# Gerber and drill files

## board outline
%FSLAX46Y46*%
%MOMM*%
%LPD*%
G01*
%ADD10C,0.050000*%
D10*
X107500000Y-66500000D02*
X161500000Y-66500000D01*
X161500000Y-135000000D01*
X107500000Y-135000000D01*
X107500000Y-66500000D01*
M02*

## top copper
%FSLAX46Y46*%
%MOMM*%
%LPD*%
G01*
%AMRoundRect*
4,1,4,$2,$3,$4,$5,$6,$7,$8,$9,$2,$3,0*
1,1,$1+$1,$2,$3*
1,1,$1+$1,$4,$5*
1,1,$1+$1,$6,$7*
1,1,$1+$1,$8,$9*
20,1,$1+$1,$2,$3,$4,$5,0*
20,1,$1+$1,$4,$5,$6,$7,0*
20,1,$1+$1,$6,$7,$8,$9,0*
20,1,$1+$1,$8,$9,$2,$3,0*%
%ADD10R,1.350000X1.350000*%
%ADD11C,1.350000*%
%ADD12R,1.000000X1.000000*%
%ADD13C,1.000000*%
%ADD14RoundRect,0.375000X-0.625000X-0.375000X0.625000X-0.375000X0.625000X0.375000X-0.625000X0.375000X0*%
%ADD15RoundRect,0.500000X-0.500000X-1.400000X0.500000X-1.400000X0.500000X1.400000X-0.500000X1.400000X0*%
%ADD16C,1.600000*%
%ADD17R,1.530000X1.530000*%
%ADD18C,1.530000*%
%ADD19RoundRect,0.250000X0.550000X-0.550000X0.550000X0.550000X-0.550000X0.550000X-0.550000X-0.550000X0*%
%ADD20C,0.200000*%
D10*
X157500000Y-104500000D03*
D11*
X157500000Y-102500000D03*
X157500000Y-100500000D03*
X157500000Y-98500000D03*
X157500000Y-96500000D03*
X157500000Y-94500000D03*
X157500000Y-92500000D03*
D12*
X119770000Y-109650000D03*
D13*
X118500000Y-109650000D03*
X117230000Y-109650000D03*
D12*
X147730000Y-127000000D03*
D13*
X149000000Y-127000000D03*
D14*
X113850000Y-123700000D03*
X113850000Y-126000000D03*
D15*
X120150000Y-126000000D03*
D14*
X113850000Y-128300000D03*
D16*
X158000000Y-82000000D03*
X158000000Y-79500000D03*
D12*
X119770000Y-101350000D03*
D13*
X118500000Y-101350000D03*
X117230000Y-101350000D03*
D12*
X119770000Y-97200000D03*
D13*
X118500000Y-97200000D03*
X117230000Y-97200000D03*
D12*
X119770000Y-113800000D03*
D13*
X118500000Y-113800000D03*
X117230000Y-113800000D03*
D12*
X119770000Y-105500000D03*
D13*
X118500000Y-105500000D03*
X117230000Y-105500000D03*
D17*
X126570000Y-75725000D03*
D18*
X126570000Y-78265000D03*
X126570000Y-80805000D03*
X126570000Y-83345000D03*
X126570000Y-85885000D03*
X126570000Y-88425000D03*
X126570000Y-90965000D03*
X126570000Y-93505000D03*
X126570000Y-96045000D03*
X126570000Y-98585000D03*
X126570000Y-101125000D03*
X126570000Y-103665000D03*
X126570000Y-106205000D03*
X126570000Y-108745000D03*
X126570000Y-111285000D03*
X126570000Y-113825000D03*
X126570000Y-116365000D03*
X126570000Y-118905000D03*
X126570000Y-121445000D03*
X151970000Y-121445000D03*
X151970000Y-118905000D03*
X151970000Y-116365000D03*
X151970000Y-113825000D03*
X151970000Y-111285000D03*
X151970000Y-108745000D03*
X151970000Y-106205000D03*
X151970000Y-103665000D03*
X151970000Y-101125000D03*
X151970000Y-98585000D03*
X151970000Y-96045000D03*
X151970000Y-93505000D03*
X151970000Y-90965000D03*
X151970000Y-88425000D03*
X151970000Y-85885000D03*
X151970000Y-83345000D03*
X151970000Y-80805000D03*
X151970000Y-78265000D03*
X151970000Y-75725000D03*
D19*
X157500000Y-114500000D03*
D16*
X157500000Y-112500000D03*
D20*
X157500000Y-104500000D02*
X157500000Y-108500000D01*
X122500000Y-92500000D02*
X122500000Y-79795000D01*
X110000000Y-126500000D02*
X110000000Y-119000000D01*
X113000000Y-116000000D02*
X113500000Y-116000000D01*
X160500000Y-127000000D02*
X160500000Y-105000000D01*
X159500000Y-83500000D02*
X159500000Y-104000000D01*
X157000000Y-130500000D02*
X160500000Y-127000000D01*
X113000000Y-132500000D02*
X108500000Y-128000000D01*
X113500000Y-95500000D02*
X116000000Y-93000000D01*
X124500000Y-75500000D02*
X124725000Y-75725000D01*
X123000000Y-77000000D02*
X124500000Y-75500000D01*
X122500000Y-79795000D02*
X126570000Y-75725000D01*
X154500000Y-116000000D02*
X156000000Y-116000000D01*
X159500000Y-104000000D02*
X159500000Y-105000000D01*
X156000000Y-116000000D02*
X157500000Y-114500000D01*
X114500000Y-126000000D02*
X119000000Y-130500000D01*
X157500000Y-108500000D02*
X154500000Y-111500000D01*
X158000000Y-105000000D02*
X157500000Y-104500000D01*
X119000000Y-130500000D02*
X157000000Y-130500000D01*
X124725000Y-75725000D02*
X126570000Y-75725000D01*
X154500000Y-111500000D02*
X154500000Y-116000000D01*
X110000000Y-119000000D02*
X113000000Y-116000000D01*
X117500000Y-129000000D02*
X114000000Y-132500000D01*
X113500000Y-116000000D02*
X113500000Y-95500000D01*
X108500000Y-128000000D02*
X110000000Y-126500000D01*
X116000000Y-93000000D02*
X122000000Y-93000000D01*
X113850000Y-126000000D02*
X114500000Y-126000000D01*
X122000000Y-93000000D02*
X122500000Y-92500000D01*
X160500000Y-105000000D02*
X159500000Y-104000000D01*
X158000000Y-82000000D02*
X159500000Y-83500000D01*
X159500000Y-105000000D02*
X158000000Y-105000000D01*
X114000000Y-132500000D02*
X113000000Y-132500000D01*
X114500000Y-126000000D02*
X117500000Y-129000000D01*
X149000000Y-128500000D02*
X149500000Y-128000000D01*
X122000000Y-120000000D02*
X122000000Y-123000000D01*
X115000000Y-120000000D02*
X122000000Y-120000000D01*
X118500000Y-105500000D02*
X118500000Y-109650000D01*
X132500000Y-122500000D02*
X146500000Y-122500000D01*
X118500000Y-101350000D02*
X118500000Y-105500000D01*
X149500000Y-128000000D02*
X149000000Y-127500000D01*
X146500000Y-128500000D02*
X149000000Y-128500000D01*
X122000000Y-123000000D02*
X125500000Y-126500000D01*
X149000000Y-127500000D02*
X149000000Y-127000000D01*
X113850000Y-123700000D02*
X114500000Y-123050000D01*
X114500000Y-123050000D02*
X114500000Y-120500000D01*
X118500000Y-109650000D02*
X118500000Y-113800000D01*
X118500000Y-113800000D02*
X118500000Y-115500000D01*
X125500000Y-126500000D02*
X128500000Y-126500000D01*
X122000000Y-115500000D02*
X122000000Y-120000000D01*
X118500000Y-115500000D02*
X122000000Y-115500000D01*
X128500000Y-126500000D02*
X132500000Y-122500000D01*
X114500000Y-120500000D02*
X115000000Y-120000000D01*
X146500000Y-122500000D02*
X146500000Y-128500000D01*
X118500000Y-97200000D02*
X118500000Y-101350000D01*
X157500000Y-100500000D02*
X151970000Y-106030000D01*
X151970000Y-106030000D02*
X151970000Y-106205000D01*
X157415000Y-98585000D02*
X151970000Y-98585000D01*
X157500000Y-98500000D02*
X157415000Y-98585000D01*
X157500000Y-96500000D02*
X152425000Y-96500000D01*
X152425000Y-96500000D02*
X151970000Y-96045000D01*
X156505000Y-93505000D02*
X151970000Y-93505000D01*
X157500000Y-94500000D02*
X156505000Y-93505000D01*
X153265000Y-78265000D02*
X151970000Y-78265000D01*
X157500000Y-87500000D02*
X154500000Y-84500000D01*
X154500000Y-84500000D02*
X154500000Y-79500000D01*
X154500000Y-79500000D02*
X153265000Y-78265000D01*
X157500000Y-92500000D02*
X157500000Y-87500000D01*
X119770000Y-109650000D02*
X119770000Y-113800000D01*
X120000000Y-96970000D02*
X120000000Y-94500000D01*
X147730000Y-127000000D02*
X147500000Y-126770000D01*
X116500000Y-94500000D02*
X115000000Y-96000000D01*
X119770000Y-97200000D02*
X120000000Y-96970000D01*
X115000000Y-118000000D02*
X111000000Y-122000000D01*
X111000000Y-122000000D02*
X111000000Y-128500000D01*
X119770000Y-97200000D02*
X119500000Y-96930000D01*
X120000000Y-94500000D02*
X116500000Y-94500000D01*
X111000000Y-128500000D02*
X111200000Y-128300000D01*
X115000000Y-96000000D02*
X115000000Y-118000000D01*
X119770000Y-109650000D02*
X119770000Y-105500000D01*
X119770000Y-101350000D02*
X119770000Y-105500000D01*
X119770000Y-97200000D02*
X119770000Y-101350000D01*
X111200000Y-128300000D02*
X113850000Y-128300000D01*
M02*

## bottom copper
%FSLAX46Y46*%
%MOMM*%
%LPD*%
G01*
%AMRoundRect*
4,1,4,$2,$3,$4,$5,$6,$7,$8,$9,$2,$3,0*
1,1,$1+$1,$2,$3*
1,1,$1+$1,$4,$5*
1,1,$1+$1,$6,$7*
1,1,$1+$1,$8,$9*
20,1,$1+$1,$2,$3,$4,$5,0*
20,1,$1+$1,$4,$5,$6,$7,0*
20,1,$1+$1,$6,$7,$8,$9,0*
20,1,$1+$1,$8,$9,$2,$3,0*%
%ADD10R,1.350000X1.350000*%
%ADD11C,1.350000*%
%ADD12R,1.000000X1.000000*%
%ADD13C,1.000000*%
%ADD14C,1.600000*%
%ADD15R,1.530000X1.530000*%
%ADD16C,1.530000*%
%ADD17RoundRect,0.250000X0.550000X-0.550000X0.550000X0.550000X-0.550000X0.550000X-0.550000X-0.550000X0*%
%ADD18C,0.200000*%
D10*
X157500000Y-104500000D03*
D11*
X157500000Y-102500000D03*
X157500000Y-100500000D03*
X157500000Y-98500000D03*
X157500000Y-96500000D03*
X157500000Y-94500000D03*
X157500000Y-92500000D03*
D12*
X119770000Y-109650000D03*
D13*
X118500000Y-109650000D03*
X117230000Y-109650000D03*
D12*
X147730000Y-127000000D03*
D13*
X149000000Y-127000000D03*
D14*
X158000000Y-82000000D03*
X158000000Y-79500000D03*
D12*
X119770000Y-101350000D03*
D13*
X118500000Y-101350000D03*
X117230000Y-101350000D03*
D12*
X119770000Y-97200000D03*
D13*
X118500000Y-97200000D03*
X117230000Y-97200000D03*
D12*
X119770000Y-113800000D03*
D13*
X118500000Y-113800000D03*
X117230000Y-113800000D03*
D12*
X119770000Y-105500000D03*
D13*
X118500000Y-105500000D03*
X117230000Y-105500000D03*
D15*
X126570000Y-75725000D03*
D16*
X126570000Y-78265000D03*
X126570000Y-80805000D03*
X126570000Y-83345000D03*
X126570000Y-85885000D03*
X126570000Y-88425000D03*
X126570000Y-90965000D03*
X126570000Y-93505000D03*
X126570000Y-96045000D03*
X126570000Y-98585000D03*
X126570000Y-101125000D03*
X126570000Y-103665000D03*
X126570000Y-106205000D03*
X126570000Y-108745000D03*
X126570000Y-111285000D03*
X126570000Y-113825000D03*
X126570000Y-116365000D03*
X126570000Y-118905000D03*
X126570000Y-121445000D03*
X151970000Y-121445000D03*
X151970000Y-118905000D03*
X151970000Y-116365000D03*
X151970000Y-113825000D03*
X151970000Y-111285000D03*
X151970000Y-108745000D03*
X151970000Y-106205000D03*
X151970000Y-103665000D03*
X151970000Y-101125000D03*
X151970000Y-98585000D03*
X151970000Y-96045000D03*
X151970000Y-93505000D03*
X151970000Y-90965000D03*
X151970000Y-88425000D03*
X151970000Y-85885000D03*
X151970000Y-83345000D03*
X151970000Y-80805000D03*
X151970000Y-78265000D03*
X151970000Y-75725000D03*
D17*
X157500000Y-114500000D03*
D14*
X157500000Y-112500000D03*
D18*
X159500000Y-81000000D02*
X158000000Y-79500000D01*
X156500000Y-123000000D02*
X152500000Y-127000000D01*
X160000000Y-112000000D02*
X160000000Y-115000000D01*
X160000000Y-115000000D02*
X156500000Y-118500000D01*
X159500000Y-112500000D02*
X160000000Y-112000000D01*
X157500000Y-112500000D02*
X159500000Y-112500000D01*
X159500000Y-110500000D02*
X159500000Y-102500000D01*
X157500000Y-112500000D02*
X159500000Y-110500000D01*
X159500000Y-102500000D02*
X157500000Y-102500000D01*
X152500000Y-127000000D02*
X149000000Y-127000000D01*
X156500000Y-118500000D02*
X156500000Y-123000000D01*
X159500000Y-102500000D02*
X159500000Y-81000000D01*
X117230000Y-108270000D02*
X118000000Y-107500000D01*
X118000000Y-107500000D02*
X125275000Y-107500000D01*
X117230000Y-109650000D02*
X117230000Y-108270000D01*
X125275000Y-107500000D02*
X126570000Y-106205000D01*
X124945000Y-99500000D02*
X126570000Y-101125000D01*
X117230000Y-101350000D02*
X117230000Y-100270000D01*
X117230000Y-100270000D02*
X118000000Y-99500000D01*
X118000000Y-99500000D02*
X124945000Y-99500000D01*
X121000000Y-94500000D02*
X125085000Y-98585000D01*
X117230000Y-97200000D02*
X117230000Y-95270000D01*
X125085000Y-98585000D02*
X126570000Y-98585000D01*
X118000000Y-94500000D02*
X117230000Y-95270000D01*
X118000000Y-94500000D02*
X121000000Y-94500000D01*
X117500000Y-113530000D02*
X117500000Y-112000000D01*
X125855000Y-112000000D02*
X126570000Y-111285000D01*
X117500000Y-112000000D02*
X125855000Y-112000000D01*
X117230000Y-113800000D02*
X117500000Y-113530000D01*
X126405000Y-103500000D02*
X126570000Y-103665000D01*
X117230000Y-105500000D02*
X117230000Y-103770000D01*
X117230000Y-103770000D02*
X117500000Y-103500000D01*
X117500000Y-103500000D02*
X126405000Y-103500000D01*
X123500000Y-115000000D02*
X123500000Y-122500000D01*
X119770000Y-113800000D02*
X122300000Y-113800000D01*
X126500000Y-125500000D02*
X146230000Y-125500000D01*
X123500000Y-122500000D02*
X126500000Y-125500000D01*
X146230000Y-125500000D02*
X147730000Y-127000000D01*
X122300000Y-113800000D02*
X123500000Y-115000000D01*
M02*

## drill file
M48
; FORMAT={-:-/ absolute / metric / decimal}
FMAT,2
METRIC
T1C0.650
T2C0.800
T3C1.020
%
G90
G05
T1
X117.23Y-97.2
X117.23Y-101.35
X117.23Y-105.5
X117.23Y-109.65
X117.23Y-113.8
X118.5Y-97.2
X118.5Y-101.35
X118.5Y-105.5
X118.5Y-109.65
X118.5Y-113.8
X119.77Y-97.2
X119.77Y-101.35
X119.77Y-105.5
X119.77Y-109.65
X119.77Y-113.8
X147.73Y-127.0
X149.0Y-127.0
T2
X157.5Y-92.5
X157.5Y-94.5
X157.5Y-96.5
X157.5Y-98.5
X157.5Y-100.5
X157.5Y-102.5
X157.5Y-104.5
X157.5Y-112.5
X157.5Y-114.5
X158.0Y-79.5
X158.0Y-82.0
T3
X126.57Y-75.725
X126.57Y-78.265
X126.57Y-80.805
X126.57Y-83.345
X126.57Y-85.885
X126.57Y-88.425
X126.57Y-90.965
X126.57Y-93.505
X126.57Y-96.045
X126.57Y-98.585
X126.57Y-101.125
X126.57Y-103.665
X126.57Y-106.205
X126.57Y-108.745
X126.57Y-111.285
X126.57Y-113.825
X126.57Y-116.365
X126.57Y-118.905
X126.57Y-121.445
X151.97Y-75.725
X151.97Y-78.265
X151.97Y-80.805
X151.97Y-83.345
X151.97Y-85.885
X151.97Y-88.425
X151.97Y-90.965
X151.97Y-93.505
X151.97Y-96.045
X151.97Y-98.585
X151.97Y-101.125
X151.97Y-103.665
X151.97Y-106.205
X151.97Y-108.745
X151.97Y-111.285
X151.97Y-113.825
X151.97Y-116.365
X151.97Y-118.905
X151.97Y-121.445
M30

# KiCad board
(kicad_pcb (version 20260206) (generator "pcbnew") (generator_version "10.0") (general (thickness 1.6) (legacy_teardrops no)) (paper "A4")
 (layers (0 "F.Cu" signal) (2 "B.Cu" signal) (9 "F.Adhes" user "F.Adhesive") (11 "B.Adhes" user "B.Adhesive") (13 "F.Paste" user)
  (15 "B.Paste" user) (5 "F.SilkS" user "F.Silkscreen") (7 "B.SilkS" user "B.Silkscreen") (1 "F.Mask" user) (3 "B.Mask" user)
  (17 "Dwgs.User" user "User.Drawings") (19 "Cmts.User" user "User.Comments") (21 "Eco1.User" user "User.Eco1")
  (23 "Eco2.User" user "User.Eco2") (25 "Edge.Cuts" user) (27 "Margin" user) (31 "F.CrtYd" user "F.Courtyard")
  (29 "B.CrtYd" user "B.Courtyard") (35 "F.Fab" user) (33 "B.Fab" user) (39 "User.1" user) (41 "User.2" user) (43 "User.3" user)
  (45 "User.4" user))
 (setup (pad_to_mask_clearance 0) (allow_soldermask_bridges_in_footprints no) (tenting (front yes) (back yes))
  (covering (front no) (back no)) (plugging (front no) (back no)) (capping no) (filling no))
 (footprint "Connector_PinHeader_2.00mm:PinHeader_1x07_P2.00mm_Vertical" (layer "F.Cu") (at 157.5 104.5 180)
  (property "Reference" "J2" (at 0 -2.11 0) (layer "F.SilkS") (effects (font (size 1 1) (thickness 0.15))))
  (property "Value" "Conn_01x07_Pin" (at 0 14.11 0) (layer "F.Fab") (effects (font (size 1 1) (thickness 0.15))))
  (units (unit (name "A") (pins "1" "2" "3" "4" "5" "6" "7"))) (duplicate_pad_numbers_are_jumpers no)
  (pad "1" thru_hole rect (at 0 0 180) (size 1.35 1.35) (drill 0.8) (layers "*.Cu" "*.Mask") (remove_unused_layers no) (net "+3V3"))
  (pad "2" thru_hole circle (at 0 2 180) (size 1.35 1.35) (drill 0.8) (layers "*.Cu" "*.Mask") (remove_unused_layers no) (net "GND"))
  (pad "3" thru_hole circle (at 0 4 180) (size 1.35 1.35) (drill 0.8) (layers "*.Cu" "*.Mask") (remove_unused_layers no)
   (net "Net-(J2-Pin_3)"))
  (pad "4" thru_hole circle (at 0 6 180) (size 1.35 1.35) (drill 0.8) (layers "*.Cu" "*.Mask") (remove_unused_layers no)
   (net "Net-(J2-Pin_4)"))
  (pad "5" thru_hole circle (at 0 8 180) (size 1.35 1.35) (drill 0.8) (layers "*.Cu" "*.Mask") (remove_unused_layers no)
   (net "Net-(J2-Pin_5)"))
  (pad "6" thru_hole circle (at 0 10 180) (size 1.35 1.35) (drill 0.8) (layers "*.Cu" "*.Mask") (remove_unused_layers no)
   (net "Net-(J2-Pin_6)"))
  (pad "7" thru_hole circle (at 0 12 180) (size 1.35 1.35) (drill 0.8) (layers "*.Cu" "*.Mask") (remove_unused_layers no)
   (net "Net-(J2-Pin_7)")))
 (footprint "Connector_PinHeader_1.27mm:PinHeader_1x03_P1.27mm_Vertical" (layer "F.Cu") (at 119.77 109.65 -90)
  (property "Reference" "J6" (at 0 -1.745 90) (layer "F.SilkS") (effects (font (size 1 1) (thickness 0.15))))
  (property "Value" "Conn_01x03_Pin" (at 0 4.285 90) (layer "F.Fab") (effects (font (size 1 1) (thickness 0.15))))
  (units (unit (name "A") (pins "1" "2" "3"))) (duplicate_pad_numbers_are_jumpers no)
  (pad "1" thru_hole rect (at 0 0 270) (size 1 1) (drill 0.65) (layers "*.Cu" "*.Mask") (remove_unused_layers no) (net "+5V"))
  (pad "2" thru_hole circle (at 0 1.27 270) (size 1 1) (drill 0.65) (layers "*.Cu" "*.Mask") (remove_unused_layers no) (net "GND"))
  (pad "3" thru_hole circle (at 0 2.54 270) (size 1 1) (drill 0.65) (layers "*.Cu" "*.Mask") (remove_unused_layers no)
   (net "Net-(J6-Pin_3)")))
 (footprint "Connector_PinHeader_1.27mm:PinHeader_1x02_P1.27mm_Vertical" (layer "F.Cu") (at 147.73 127 90)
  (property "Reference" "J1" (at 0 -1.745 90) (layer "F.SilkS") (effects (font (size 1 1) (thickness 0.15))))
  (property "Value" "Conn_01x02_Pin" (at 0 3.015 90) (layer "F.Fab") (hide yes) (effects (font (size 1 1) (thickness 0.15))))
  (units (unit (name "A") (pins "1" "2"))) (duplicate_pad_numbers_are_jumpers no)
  (pad "1" thru_hole rect (at 0 0 90) (size 1 1) (drill 0.65) (layers "*.Cu" "*.Mask") (remove_unused_layers no) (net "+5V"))
  (pad "2" thru_hole circle (at 0 1.27 90) (size 1 1) (drill 0.65) (layers "*.Cu" "*.Mask") (remove_unused_layers no) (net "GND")))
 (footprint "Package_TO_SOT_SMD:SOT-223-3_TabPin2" (layer "F.Cu") (at 117 126)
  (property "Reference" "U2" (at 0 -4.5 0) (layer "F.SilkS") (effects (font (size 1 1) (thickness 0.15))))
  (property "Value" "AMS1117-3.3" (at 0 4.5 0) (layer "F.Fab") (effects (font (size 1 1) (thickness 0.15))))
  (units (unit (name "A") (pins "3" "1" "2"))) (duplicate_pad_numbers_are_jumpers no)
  (pad "1" smd roundrect (at -3.15 -2.3) (size 2 1.5) (layers "F.Cu" "F.Mask" "F.Paste") (roundrect_rratio 0.25) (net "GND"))
  (pad "2" smd roundrect (at -3.15 0) (size 2 1.5) (layers "F.Cu" "F.Mask" "F.Paste") (roundrect_rratio 0.25) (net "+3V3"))
  (pad "2" smd roundrect (at 3.15 0) (size 2 3.8) (layers "F.Cu" "F.Mask" "F.Paste") (roundrect_rratio 0.25) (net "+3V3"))
  (pad "3" smd roundrect (at -3.15 2.3) (size 2 1.5) (layers "F.Cu" "F.Mask" "F.Paste") (roundrect_rratio 0.25) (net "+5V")))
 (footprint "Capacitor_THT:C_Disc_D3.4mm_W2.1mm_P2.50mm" (layer "F.Cu") (at 158 82 90)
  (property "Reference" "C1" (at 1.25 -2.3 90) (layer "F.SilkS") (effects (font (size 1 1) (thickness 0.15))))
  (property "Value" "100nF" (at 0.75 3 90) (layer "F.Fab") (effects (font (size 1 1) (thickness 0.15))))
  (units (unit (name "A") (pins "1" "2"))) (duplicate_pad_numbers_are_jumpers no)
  (pad "1" thru_hole circle (at 0 0 90) (size 1.6 1.6) (drill 0.8) (layers "*.Cu" "*.Mask") (remove_unused_layers no) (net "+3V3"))
  (pad "2" thru_hole circle (at 2.5 0 90) (size 1.6 1.6) (drill 0.8) (layers "*.Cu" "*.Mask") (remove_unused_layers no) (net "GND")))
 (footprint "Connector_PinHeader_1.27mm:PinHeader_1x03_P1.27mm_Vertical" (layer "F.Cu") (at 119.77 101.35 -90)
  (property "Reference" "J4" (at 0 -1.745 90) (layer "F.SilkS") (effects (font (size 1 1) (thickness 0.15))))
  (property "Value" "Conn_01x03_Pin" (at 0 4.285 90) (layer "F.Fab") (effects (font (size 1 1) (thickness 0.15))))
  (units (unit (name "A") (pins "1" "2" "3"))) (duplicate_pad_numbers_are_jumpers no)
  (pad "1" thru_hole rect (at 0 0 270) (size 1 1) (drill 0.65) (layers "*.Cu" "*.Mask") (remove_unused_layers no) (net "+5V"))
  (pad "2" thru_hole circle (at 0 1.27 270) (size 1 1) (drill 0.65) (layers "*.Cu" "*.Mask") (remove_unused_layers no) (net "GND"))
  (pad "3" thru_hole circle (at 0 2.54 270) (size 1 1) (drill 0.65) (layers "*.Cu" "*.Mask") (remove_unused_layers no)
   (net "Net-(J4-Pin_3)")))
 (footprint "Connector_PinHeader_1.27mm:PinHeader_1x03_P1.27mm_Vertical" (layer "F.Cu") (at 119.77 97.2 -90)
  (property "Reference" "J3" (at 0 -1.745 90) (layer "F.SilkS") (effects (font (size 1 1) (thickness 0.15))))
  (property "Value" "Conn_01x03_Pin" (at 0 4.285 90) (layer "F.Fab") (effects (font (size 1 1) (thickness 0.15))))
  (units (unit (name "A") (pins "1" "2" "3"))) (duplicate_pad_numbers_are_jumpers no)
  (pad "1" thru_hole rect (at 0 0 270) (size 1 1) (drill 0.65) (layers "*.Cu" "*.Mask") (remove_unused_layers no) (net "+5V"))
  (pad "2" thru_hole circle (at 0 1.27 270) (size 1 1) (drill 0.65) (layers "*.Cu" "*.Mask") (remove_unused_layers no) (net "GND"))
  (pad "3" thru_hole circle (at 0 2.54 270) (size 1 1) (drill 0.65) (layers "*.Cu" "*.Mask") (remove_unused_layers no)
   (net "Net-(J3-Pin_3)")))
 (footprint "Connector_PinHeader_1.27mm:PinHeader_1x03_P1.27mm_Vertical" (layer "F.Cu") (at 119.77 113.8 -90)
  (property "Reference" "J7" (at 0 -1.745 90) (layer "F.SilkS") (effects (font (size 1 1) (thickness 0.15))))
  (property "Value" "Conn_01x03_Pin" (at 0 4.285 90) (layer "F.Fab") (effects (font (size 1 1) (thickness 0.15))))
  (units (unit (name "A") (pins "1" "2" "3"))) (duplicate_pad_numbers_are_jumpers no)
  (pad "1" thru_hole rect (at 0 0 270) (size 1 1) (drill 0.65) (layers "*.Cu" "*.Mask") (remove_unused_layers no) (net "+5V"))
  (pad "2" thru_hole circle (at 0 1.27 270) (size 1 1) (drill 0.65) (layers "*.Cu" "*.Mask") (remove_unused_layers no) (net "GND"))
  (pad "3" thru_hole circle (at 0 2.54 270) (size 1 1) (drill 0.65) (layers "*.Cu" "*.Mask") (remove_unused_layers no)
   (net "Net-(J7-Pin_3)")))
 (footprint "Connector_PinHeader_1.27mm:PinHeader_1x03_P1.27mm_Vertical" (layer "F.Cu") (at 119.77 105.5 -90)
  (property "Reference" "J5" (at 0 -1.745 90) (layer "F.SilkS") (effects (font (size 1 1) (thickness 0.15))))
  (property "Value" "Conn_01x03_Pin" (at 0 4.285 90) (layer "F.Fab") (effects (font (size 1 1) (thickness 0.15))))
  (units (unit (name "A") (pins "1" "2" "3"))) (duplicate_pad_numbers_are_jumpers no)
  (pad "1" thru_hole rect (at 0 0 270) (size 1 1) (drill 0.65) (layers "*.Cu" "*.Mask") (remove_unused_layers no) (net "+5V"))
  (pad "2" thru_hole circle (at 0 1.27 270) (size 1 1) (drill 0.65) (layers "*.Cu" "*.Mask") (remove_unused_layers no) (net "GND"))
  (pad "3" thru_hole circle (at 0 2.54 270) (size 1 1) (drill 0.65) (layers "*.Cu" "*.Mask") (remove_unused_layers no)
   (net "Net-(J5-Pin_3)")))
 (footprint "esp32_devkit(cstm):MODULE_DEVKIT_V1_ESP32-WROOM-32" (layer "F.Cu") (at 139.27 98.575)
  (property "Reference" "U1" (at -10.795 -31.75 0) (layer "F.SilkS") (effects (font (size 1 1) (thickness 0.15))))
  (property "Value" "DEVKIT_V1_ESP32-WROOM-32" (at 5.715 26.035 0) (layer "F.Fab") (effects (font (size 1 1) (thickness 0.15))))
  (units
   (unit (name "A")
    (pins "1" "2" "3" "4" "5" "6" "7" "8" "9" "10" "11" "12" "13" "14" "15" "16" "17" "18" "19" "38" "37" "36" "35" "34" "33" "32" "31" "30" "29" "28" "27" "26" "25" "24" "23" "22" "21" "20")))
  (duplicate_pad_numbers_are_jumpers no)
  (pad "1" thru_hole rect (at -12.7 -22.85) (size 1.53 1.53) (drill 1.02) (layers "*.Cu" "*.Mask") (remove_unused_layers no) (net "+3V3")
   (solder_mask_margin 0.102))
  (pad "2" thru_hole circle (at -12.7 -20.31) (size 1.53 1.53) (drill 1.02) (layers "*.Cu" "*.Mask") (remove_unused_layers no)
   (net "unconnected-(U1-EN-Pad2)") (solder_mask_margin 0.102))
  (pad "3" thru_hole circle (at -12.7 -17.77) (size 1.53 1.53) (drill 1.02) (layers "*.Cu" "*.Mask") (remove_unused_layers no)
   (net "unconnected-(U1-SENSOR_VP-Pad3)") (solder_mask_margin 0.102))
  (pad "4" thru_hole circle (at -12.7 -15.23) (size 1.53 1.53) (drill 1.02) (layers "*.Cu" "*.Mask") (remove_unused_layers no)
   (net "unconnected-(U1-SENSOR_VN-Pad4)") (solder_mask_margin 0.102))
  (pad "5" thru_hole circle (at -12.7 -12.69) (size 1.53 1.53) (drill 1.02) (layers "*.Cu" "*.Mask") (remove_unused_layers no)
   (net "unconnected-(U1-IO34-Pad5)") (solder_mask_margin 0.102))
  (pad "6" thru_hole circle (at -12.7 -10.15) (size 1.53 1.53) (drill 1.02) (layers "*.Cu" "*.Mask") (remove_unused_layers no)
   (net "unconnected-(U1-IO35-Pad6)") (solder_mask_margin 0.102))
  (pad "7" thru_hole circle (at -12.7 -7.61) (size 1.53 1.53) (drill 1.02) (layers "*.Cu" "*.Mask") (remove_unused_layers no)
   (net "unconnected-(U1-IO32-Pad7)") (solder_mask_margin 0.102))
  (pad "8" thru_hole circle (at -12.7 -5.07) (size 1.53 1.53) (drill 1.02) (layers "*.Cu" "*.Mask") (remove_unused_layers no)
   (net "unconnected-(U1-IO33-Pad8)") (solder_mask_margin 0.102))
  (pad "9" thru_hole circle (at -12.7 -2.53) (size 1.53 1.53) (drill 1.02) (layers "*.Cu" "*.Mask") (remove_unused_layers no)
   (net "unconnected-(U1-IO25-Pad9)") (solder_mask_margin 0.102))
  (pad "10" thru_hole circle (at -12.7 0.01) (size 1.53 1.53) (drill 1.02) (layers "*.Cu" "*.Mask") (remove_unused_layers no)
   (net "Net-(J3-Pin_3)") (solder_mask_margin 0.102))
  (pad "11" thru_hole circle (at -12.7 2.55) (size 1.53 1.53) (drill 1.02) (layers "*.Cu" "*.Mask") (remove_unused_layers no)
   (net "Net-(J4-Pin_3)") (solder_mask_margin 0.102))
  (pad "12" thru_hole circle (at -12.7 5.09) (size 1.53 1.53) (drill 1.02) (layers "*.Cu" "*.Mask") (remove_unused_layers no)
   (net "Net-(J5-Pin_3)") (solder_mask_margin 0.102))
  (pad "13" thru_hole circle (at -12.7 7.63) (size 1.53 1.53) (drill 1.02) (layers "*.Cu" "*.Mask") (remove_unused_layers no)
   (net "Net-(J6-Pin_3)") (solder_mask_margin 0.102))
  (pad "14" thru_hole circle (at -12.7 10.17) (size 1.53 1.53) (drill 1.02) (layers "*.Cu" "*.Mask") (remove_unused_layers no) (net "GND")
   (solder_mask_margin 0.102))
  (pad "15" thru_hole circle (at -12.7 12.71) (size 1.53 1.53) (drill 1.02) (layers "*.Cu" "*.Mask") (remove_unused_layers no)
   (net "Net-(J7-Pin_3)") (solder_mask_margin 0.102))
  (pad "16" thru_hole circle (at -12.7 15.25) (size 1.53 1.53) (drill 1.02) (layers "*.Cu" "*.Mask") (remove_unused_layers no)
   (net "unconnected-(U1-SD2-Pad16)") (solder_mask_margin 0.102))
  (pad "17" thru_hole circle (at -12.7 17.79) (size 1.53 1.53) (drill 1.02) (layers "*.Cu" "*.Mask") (remove_unused_layers no)
   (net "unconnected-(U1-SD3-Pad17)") (solder_mask_margin 0.102))
  (pad "18" thru_hole circle (at -12.7 20.33) (size 1.53 1.53) (drill 1.02) (layers "*.Cu" "*.Mask") (remove_unused_layers no)
   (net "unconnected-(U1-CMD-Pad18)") (solder_mask_margin 0.102))
  (pad "19" thru_hole circle (at -12.7 22.87) (size 1.53 1.53) (drill 1.02) (layers "*.Cu" "*.Mask") (remove_unused_layers no)
   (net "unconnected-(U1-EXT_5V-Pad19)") (solder_mask_margin 0.102))
  (pad "20" thru_hole circle (at 12.7 22.87) (size 1.53 1.53) (drill 1.02) (layers "*.Cu" "*.Mask") (remove_unused_layers no)
   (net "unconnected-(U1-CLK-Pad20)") (solder_mask_margin 0.102))
  (pad "21" thru_hole circle (at 12.7 20.33) (size 1.53 1.53) (drill 1.02) (layers "*.Cu" "*.Mask") (remove_unused_layers no)
   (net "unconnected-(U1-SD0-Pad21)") (solder_mask_margin 0.102))
  (pad "22" thru_hole circle (at 12.7 17.79) (size 1.53 1.53) (drill 1.02) (layers "*.Cu" "*.Mask") (remove_unused_layers no)
   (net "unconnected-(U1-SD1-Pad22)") (solder_mask_margin 0.102))
  (pad "23" thru_hole circle (at 12.7 15.25) (size 1.53 1.53) (drill 1.02) (layers "*.Cu" "*.Mask") (remove_unused_layers no)
   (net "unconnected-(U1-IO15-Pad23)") (solder_mask_margin 0.102))
  (pad "24" thru_hole circle (at 12.7 12.71) (size 1.53 1.53) (drill 1.02) (layers "*.Cu" "*.Mask") (remove_unused_layers no)
   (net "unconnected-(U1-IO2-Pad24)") (solder_mask_margin 0.102))
  (pad "25" thru_hole circle (at 12.7 10.17) (size 1.53 1.53) (drill 1.02) (layers "*.Cu" "*.Mask") (remove_unused_layers no)
   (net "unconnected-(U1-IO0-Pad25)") (solder_mask_margin 0.102))
  (pad "26" thru_hole circle (at 12.7 7.63) (size 1.53 1.53) (drill 1.02) (layers "*.Cu" "*.Mask") (remove_unused_layers no)
   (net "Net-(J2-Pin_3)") (solder_mask_margin 0.102))
  (pad "27" thru_hole circle (at 12.7 5.09) (size 1.53 1.53) (drill 1.02) (layers "*.Cu" "*.Mask") (remove_unused_layers no)
   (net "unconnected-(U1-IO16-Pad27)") (solder_mask_margin 0.102))
  (pad "28" thru_hole circle (at 12.7 2.55) (size 1.53 1.53) (drill 1.02) (layers "*.Cu" "*.Mask") (remove_unused_layers no)
   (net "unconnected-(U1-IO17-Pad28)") (solder_mask_margin 0.102))
  (pad "29" thru_hole circle (at 12.7 0.01) (size 1.53 1.53) (drill 1.02) (layers "*.Cu" "*.Mask") (remove_unused_layers no)
   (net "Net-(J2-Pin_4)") (solder_mask_margin 0.102))
  (pad "30" thru_hole circle (at 12.7 -2.53) (size 1.53 1.53) (drill 1.02) (layers "*.Cu" "*.Mask") (remove_unused_layers no)
   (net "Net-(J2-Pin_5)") (solder_mask_margin 0.102))
  (pad "31" thru_hole circle (at 12.7 -5.07) (size 1.53 1.53) (drill 1.02) (layers "*.Cu" "*.Mask") (remove_unused_layers no)
   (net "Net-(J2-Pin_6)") (solder_mask_margin 0.102))
  (pad "32" thru_hole circle (at 12.7 -7.61) (size 1.53 1.53) (drill 1.02) (layers "*.Cu" "*.Mask") (remove_unused_layers no)
   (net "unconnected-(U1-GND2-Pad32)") (solder_mask_margin 0.102))
  (pad "33" thru_hole circle (at 12.7 -10.15) (size 1.53 1.53) (drill 1.02) (layers "*.Cu" "*.Mask") (remove_unused_layers no)
   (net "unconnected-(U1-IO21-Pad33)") (solder_mask_margin 0.102))
  (pad "34" thru_hole circle (at 12.7 -12.69) (size 1.53 1.53) (drill 1.02) (layers "*.Cu" "*.Mask") (remove_unused_layers no)
   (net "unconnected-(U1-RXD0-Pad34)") (solder_mask_margin 0.102))
  (pad "35" thru_hole circle (at 12.7 -15.23) (size 1.53 1.53) (drill 1.02) (layers "*.Cu" "*.Mask") (remove_unused_layers no)
   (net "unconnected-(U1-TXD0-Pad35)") (solder_mask_margin 0.102))
  (pad "36" thru_hole circle (at 12.7 -17.77) (size 1.53 1.53) (drill 1.02) (layers "*.Cu" "*.Mask") (remove_unused_layers no)
   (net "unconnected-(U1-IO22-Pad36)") (solder_mask_margin 0.102))
  (pad "37" thru_hole circle (at 12.7 -20.31) (size 1.53 1.53) (drill 1.02) (layers "*.Cu" "*.Mask") (remove_unused_layers no)
   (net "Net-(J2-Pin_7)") (solder_mask_margin 0.102))
  (pad "38" thru_hole circle (at 12.7 -22.85) (size 1.53 1.53) (drill 1.02) (layers "*.Cu" "*.Mask") (remove_unused_layers no) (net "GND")
   (solder_mask_margin 0.102)))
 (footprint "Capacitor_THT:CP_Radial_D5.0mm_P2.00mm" (layer "F.Cu") (at 157.5 114.5 90)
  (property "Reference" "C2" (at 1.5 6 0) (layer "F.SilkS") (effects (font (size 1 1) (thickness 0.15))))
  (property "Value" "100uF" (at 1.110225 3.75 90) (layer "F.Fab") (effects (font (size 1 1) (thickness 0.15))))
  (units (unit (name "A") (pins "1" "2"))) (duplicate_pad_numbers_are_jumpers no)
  (pad "1" thru_hole roundrect (at 0 0 90) (size 1.6 1.6) (drill 0.8) (layers "*.Cu" "*.Mask") (remove_unused_layers no)
   (roundrect_rratio 0.15625) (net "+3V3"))
  (pad "2" thru_hole circle (at 2 0 90) (size 1.6 1.6) (drill 0.8) (layers "*.Cu" "*.Mask") (remove_unused_layers no) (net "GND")))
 (gr_rect (start 107.5 66.5) (end 161.5 135) (stroke (width 0.05) (type default)) (fill no) (layer "Edge.Cuts"))
 (segment (start 157.5 104.5) (end 157.5 108.5) (width 0.2) (layer "F.Cu") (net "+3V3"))
 (segment (start 122.5 92.5) (end 122.5 79.795) (width 0.2) (layer "F.Cu") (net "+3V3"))
 (segment (start 110 126.5) (end 110 119) (width 0.2) (layer "F.Cu") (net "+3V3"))
 (segment (start 113 116) (end 113.5 116) (width 0.2) (layer "F.Cu") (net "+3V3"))
 (segment (start 160.5 127) (end 160.5 105) (width 0.2) (layer "F.Cu") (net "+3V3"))
 (segment (start 159.5 83.5) (end 159.5 104) (width 0.2) (layer "F.Cu") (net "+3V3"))
 (segment (start 157 130.5) (end 160.5 127) (width 0.2) (layer "F.Cu") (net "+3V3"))
 (segment (start 113 132.5) (end 108.5 128) (width 0.2) (layer "F.Cu") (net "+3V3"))
 (segment (start 113.5 95.5) (end 116 93) (width 0.2) (layer "F.Cu") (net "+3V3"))
 (segment (start 124.5 75.5) (end 124.725 75.725) (width 0.2) (layer "F.Cu") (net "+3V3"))
 (segment (start 123 77) (end 124.5 75.5) (width 0.2) (layer "F.Cu") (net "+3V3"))
 (segment (start 122.5 79.795) (end 126.57 75.725) (width 0.2) (layer "F.Cu") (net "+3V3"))
 (segment (start 154.5 116) (end 156 116) (width 0.2) (layer "F.Cu") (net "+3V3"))
 (segment (start 159.5 104) (end 159.5 105) (width 0.2) (layer "F.Cu") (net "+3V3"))
 (segment (start 156 116) (end 157.5 114.5) (width 0.2) (layer "F.Cu") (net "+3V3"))
 (segment (start 114.5 126) (end 119 130.5) (width 0.2) (layer "F.Cu") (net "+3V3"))
 (segment (start 157.5 108.5) (end 154.5 111.5) (width 0.2) (layer "F.Cu") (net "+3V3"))
 (segment (start 158 105) (end 157.5 104.5) (width 0.2) (layer "F.Cu") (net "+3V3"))
 (segment (start 119 130.5) (end 157 130.5) (width 0.2) (layer "F.Cu") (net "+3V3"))
 (segment (start 124.725 75.725) (end 126.57 75.725) (width 0.2) (layer "F.Cu") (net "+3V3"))
 (segment (start 154.5 111.5) (end 154.5 116) (width 0.2) (layer "F.Cu") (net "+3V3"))
 (segment (start 110 119) (end 113 116) (width 0.2) (layer "F.Cu") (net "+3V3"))
 (segment (start 117.5 129) (end 114 132.5) (width 0.2) (layer "F.Cu") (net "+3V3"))
 (segment (start 113.5 116) (end 113.5 95.5) (width 0.2) (layer "F.Cu") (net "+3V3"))
 (segment (start 108.5 128) (end 110 126.5) (width 0.2) (layer "F.Cu") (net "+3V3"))
 (segment (start 116 93) (end 122 93) (width 0.2) (layer "F.Cu") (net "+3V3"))
 (segment (start 113.85 126) (end 114.5 126) (width 0.2) (layer "F.Cu") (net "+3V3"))
 (segment (start 122 93) (end 122.5 92.5) (width 0.2) (layer "F.Cu") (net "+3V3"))
 (segment (start 160.5 105) (end 159.5 104) (width 0.2) (layer "F.Cu") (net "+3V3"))
 (segment (start 158 82) (end 159.5 83.5) (width 0.2) (layer "F.Cu") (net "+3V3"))
 (segment (start 159.5 105) (end 158 105) (width 0.2) (layer "F.Cu") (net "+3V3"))
 (segment (start 114 132.5) (end 113 132.5) (width 0.2) (layer "F.Cu") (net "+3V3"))
 (segment (start 114.5 126) (end 117.5 129) (width 0.2) (layer "F.Cu") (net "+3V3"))
 (segment (start 149 128.5) (end 149.5 128) (width 0.2) (layer "F.Cu") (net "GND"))
 (segment (start 122 120) (end 122 123) (width 0.2) (layer "F.Cu") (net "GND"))
 (segment (start 115 120) (end 122 120) (width 0.2) (layer "F.Cu") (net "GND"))
 (segment (start 118.5 105.5) (end 118.5 109.65) (width 0.2) (layer "F.Cu") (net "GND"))
 (segment (start 132.5 122.5) (end 146.5 122.5) (width 0.2) (layer "F.Cu") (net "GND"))
 (segment (start 118.5 101.35) (end 118.5 105.5) (width 0.2) (layer "F.Cu") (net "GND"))
 (segment (start 149.5 128) (end 149 127.5) (width 0.2) (layer "F.Cu") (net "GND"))
 (segment (start 146.5 128.5) (end 149 128.5) (width 0.2) (layer "F.Cu") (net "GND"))
 (segment (start 122 123) (end 125.5 126.5) (width 0.2) (layer "F.Cu") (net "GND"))
 (segment (start 149 127.5) (end 149 127) (width 0.2) (layer "F.Cu") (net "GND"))
 (segment (start 113.85 123.7) (end 114.5 123.05) (width 0.2) (layer "F.Cu") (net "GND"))
 (segment (start 114.5 123.05) (end 114.5 120.5) (width 0.2) (layer "F.Cu") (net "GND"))
 (segment (start 118.5 109.65) (end 118.5 113.8) (width 0.2) (layer "F.Cu") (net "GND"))
 (segment (start 118.5 113.8) (end 118.5 115.5) (width 0.2) (layer "F.Cu") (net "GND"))
 (segment (start 125.5 126.5) (end 128.5 126.5) (width 0.2) (layer "F.Cu") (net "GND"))
 (segment (start 122 115.5) (end 122 120) (width 0.2) (layer "F.Cu") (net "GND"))
 (segment (start 118.5 115.5) (end 122 115.5) (width 0.2) (layer "F.Cu") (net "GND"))
 (segment (start 128.5 126.5) (end 132.5 122.5) (width 0.2) (layer "F.Cu") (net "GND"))
 (segment (start 114.5 120.5) (end 115 120) (width 0.2) (layer "F.Cu") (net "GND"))
 (segment (start 146.5 122.5) (end 146.5 128.5) (width 0.2) (layer "F.Cu") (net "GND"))
 (segment (start 118.5 97.2) (end 118.5 101.35) (width 0.2) (layer "F.Cu") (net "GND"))
 (segment (start 159.5 81) (end 158 79.5) (width 0.2) (layer "B.Cu") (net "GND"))
 (segment (start 156.5 123) (end 152.5 127) (width 0.2) (layer "B.Cu") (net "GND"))
 (segment (start 160 112) (end 160 115) (width 0.2) (layer "B.Cu") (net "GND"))
 (segment (start 160 115) (end 156.5 118.5) (width 0.2) (layer "B.Cu") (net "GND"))
 (segment (start 159.5 112.5) (end 160 112) (width 0.2) (layer "B.Cu") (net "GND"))
 (segment (start 157.5 112.5) (end 159.5 112.5) (width 0.2) (layer "B.Cu") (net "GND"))
 (segment (start 159.5 110.5) (end 159.5 102.5) (width 0.2) (layer "B.Cu") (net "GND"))
 (segment (start 157.5 112.5) (end 159.5 110.5) (width 0.2) (layer "B.Cu") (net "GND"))
 (segment (start 159.5 102.5) (end 157.5 102.5) (width 0.2) (layer "B.Cu") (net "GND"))
 (segment (start 152.5 127) (end 149 127) (width 0.2) (layer "B.Cu") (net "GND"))
 (segment (start 156.5 118.5) (end 156.5 123) (width 0.2) (layer "B.Cu") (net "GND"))
 (segment (start 159.5 102.5) (end 159.5 81) (width 0.2) (layer "B.Cu") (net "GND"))
 (segment (start 157.5 100.5) (end 151.97 106.03) (width 0.2) (layer "F.Cu") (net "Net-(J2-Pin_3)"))
 (segment (start 151.97 106.03) (end 151.97 106.205) (width 0.2) (layer "F.Cu") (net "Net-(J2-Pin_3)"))
 (segment (start 157.415 98.585) (end 151.97 98.585) (width 0.2) (layer "F.Cu") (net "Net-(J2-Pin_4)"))
 (segment (start 157.5 98.5) (end 157.415 98.585) (width 0.2) (layer "F.Cu") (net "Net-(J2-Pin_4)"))
 (segment (start 157.5 96.5) (end 152.425 96.5) (width 0.2) (layer "F.Cu") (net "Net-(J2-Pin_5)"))
 (segment (start 152.425 96.5) (end 151.97 96.045) (width 0.2) (layer "F.Cu") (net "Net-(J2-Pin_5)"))
 (segment (start 156.505 93.505) (end 151.97 93.505) (width 0.2) (layer "F.Cu") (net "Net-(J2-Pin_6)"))
 (segment (start 157.5 94.5) (end 156.505 93.505) (width 0.2) (layer "F.Cu") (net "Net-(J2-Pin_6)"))
 (segment (start 153.265 78.265) (end 151.97 78.265) (width 0.2) (layer "F.Cu") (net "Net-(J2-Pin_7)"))
 (segment (start 157.5 87.5) (end 154.5 84.5) (width 0.2) (layer "F.Cu") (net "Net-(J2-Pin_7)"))
 (segment (start 154.5 84.5) (end 154.5 79.5) (width 0.2) (layer "F.Cu") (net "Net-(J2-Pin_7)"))
 (segment (start 154.5 79.5) (end 153.265 78.265) (width 0.2) (layer "F.Cu") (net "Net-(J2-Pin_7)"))
 (segment (start 157.5 92.5) (end 157.5 87.5) (width 0.2) (layer "F.Cu") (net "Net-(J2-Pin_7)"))
 (segment (start 117.23 108.27) (end 118 107.5) (width 0.2) (layer "B.Cu") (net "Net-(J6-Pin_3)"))
 (segment (start 118 107.5) (end 125.275 107.5) (width 0.2) (layer "B.Cu") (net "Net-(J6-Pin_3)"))
 (segment (start 117.23 109.65) (end 117.23 108.27) (width 0.2) (layer "B.Cu") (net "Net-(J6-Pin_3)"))
 (segment (start 125.275 107.5) (end 126.57 106.205) (width 0.2) (layer "B.Cu") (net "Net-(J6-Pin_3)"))
 (segment (start 124.945 99.5) (end 126.57 101.125) (width 0.2) (layer "B.Cu") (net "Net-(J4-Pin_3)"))
 (segment (start 117.23 101.35) (end 117.23 100.27) (width 0.2) (layer "B.Cu") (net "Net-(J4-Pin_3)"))
 (segment (start 117.23 100.27) (end 118 99.5) (width 0.2) (layer "B.Cu") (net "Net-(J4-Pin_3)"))
 (segment (start 118 99.5) (end 124.945 99.5) (width 0.2) (layer "B.Cu") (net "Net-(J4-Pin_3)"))
 (segment (start 121 94.5) (end 125.085 98.585) (width 0.2) (layer "B.Cu") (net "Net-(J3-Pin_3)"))
 (segment (start 117.23 97.2) (end 117.23 95.27) (width 0.2) (layer "B.Cu") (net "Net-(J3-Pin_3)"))
 (segment (start 125.085 98.585) (end 126.57 98.585) (width 0.2) (layer "B.Cu") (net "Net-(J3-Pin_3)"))
 (segment (start 118 94.5) (end 117.23 95.27) (width 0.2) (layer "B.Cu") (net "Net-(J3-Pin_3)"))
 (segment (start 118 94.5) (end 121 94.5) (width 0.2) (layer "B.Cu") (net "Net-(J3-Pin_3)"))
 (segment (start 117.5 113.53) (end 117.5 112) (width 0.2) (layer "B.Cu") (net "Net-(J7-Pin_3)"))
 (segment (start 125.855 112) (end 126.57 111.285) (width 0.2) (layer "B.Cu") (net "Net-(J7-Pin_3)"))
 (segment (start 117.5 112) (end 125.855 112) (width 0.2) (layer "B.Cu") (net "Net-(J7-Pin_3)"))
 (segment (start 117.23 113.8) (end 117.5 113.53) (width 0.2) (layer "B.Cu") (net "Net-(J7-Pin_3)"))
 (segment (start 126.405 103.5) (end 126.57 103.665) (width 0.2) (layer "B.Cu") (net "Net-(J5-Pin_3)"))
 (segment (start 117.23 105.5) (end 117.23 103.77) (width 0.2) (layer "B.Cu") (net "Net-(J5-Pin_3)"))
 (segment (start 117.23 103.77) (end 117.5 103.5) (width 0.2) (layer "B.Cu") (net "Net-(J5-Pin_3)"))
 (segment (start 117.5 103.5) (end 126.405 103.5) (width 0.2) (layer "B.Cu") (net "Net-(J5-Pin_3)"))
 (segment (start 119.77 109.65) (end 119.77 113.8) (width 0.2) (layer "F.Cu") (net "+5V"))
 (segment (start 120 96.97) (end 120 94.5) (width 0.2) (layer "F.Cu") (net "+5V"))
 (segment (start 147.73 127) (end 147.5 126.77) (width 0.2) (layer "F.Cu") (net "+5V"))
 (segment (start 116.5 94.5) (end 115 96) (width 0.2) (layer "F.Cu") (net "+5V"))
 (segment (start 119.77 97.2) (end 120 96.97) (width 0.2) (layer "F.Cu") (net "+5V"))
 (segment (start 115 118) (end 111 122) (width 0.2) (layer "F.Cu") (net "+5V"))
 (segment (start 111 122) (end 111 128.5) (width 0.2) (layer "F.Cu") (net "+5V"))
 (segment (start 119.77 97.2) (end 119.5 96.93) (width 0.2) (layer "F.Cu") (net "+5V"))
 (segment (start 120 94.5) (end 116.5 94.5) (width 0.2) (layer "F.Cu") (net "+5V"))
 (segment (start 111 128.5) (end 111.2 128.3) (width 0.2) (layer "F.Cu") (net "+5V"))
 (segment (start 115 96) (end 115 118) (width 0.2) (layer "F.Cu") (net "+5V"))
 (segment (start 119.77 109.65) (end 119.77 105.5) (width 0.2) (layer "F.Cu") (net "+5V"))
 (segment (start 119.77 101.35) (end 119.77 105.5) (width 0.2) (layer "F.Cu") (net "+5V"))
 (segment (start 119.77 97.2) (end 119.77 101.35) (width 0.2) (layer "F.Cu") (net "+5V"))
 (segment (start 111.2 128.3) (end 113.85 128.3) (width 0.2) (layer "F.Cu") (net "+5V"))
 (segment (start 123.5 115) (end 123.5 122.5) (width 0.2) (layer "B.Cu") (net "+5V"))
 (segment (start 119.77 113.8) (end 122.3 113.8) (width 0.2) (layer "B.Cu") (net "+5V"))
 (segment (start 126.5 125.5) (end 146.23 125.5) (width 0.2) (layer "B.Cu") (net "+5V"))
 (segment (start 123.5 122.5) (end 126.5 125.5) (width 0.2) (layer "B.Cu") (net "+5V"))
 (segment (start 146.23 125.5) (end 147.73 127) (width 0.2) (layer "B.Cu") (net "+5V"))
 (segment (start 122.3 113.8) (end 123.5 115) (width 0.2) (layer "B.Cu") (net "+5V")))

